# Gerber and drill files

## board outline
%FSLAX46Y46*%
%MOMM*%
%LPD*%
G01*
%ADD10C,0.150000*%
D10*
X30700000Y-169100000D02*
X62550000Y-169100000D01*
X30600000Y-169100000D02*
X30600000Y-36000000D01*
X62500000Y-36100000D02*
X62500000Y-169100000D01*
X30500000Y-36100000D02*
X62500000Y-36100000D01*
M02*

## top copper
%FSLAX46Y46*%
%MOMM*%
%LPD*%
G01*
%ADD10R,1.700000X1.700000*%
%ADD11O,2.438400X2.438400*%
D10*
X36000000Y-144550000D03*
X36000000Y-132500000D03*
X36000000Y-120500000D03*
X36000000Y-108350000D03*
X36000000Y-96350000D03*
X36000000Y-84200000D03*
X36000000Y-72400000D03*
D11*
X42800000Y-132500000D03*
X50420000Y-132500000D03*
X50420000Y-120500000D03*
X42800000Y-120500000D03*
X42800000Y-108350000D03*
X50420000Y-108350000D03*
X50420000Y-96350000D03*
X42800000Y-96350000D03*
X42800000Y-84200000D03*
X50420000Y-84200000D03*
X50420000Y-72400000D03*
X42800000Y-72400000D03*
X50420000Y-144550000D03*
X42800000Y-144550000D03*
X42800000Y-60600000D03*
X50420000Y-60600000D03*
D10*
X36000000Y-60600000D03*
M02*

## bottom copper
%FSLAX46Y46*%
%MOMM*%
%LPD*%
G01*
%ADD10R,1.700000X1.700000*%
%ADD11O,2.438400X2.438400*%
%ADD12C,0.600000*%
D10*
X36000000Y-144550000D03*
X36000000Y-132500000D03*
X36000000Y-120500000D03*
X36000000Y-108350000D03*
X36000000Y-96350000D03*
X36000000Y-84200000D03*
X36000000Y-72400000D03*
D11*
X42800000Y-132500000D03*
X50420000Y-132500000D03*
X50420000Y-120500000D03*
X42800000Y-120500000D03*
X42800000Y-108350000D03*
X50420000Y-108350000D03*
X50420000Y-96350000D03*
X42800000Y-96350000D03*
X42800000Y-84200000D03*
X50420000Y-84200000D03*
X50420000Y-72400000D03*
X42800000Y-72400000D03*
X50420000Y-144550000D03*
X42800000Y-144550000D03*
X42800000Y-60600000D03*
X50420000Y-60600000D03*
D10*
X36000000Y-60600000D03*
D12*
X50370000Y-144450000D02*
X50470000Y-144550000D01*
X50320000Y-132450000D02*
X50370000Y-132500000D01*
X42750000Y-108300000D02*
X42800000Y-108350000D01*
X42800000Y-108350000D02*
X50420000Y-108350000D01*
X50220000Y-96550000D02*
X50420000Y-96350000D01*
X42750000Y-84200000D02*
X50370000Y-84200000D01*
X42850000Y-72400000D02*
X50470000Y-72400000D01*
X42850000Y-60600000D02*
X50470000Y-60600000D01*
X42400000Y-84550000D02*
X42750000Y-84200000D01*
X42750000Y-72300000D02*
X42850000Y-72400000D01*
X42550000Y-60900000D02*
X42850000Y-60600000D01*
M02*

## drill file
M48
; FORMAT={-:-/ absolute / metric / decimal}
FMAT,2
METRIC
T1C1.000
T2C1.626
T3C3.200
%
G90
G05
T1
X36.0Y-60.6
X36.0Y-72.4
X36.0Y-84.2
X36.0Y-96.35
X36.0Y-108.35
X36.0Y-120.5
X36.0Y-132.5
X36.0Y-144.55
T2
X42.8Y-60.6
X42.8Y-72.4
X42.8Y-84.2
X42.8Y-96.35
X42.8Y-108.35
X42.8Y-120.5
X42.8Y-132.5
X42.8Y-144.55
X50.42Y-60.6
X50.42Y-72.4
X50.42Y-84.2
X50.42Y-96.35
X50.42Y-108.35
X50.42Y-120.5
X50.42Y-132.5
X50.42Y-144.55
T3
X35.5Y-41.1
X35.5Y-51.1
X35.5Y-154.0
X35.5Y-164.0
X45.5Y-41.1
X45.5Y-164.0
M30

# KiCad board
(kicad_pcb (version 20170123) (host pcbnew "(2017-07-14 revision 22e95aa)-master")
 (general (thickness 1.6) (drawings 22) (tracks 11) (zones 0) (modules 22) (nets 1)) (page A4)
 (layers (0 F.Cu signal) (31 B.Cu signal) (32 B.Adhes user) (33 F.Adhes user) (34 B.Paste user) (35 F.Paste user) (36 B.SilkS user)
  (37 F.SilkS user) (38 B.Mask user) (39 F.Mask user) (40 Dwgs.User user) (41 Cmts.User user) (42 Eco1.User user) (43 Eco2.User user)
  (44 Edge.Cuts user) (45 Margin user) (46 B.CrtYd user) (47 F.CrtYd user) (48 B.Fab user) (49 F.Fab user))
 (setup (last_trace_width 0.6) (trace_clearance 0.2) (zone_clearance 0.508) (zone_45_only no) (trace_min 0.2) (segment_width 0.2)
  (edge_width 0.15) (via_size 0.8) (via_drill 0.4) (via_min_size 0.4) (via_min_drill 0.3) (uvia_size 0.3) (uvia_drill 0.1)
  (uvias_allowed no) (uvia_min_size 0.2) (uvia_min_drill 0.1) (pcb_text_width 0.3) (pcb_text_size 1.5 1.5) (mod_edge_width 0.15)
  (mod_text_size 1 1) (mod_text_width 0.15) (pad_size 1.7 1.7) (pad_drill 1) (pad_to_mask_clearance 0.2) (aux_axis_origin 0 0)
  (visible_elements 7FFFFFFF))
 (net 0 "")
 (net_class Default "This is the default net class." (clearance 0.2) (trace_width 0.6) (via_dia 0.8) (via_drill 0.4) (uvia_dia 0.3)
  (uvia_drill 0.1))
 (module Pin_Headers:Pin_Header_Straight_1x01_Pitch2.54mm (layer F.Cu) (at 36 144.55)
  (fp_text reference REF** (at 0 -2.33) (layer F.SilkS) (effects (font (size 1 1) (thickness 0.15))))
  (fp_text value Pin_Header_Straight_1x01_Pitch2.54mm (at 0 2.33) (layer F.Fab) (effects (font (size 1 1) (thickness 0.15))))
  (pad 1 thru_hole rect (at 0 0) (size 1.7 1.7) (drill 1) (layers *.Cu *.Mask)))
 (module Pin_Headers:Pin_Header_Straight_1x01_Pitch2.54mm (layer F.Cu) (at 36 132.5)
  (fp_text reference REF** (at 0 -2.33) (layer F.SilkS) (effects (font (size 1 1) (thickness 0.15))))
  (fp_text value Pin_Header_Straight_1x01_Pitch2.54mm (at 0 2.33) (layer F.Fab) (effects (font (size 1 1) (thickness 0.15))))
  (pad 1 thru_hole rect (at 0 0) (size 1.7 1.7) (drill 1) (layers *.Cu *.Mask)))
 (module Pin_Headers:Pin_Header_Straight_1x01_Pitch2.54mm (layer F.Cu) (at 36 120.5)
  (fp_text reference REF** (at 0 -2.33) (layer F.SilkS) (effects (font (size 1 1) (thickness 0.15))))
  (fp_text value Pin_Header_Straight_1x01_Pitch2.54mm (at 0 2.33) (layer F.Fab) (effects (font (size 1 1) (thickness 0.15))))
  (pad 1 thru_hole rect (at 0 0) (size 1.7 1.7) (drill 1) (layers *.Cu *.Mask)))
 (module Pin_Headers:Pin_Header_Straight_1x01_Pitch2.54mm (layer F.Cu) (at 36 108.35)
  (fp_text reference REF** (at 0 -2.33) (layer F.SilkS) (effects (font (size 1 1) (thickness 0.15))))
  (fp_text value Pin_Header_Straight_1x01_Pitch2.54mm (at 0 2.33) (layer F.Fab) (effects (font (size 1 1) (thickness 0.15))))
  (pad 1 thru_hole rect (at 0 0) (size 1.7 1.7) (drill 1) (layers *.Cu *.Mask)))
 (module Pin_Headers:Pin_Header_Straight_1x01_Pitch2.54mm (layer F.Cu) (at 36 96.35)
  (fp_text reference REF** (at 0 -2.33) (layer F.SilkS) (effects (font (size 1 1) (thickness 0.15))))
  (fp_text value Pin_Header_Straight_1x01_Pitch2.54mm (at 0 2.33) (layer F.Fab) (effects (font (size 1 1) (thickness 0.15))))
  (pad 1 thru_hole rect (at 0 0) (size 1.7 1.7) (drill 1) (layers *.Cu *.Mask)))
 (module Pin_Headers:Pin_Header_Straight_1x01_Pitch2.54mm (layer F.Cu) (at 36 84.2)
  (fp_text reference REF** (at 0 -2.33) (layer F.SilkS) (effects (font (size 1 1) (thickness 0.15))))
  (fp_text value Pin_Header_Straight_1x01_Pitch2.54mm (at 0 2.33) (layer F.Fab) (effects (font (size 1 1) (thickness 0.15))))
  (pad 1 thru_hole rect (at 0 0) (size 1.7 1.7) (drill 1) (layers *.Cu *.Mask)))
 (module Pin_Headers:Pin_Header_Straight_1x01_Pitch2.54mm (layer F.Cu) (at 36 72.4)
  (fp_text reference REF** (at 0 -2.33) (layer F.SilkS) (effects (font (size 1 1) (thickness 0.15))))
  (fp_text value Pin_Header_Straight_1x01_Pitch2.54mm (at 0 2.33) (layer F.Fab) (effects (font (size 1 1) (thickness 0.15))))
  (pad 1 thru_hole rect (at 0 0) (size 1.7 1.7) (drill 1) (layers *.Cu *.Mask)))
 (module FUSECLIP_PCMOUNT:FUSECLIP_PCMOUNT (layer F.Cu) (at 42.8 132.5)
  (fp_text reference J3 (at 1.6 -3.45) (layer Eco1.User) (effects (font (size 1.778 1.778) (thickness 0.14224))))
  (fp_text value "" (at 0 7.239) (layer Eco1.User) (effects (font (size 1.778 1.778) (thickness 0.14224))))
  (pad 1 thru_hole oval (at 0 0) (size 2.4384 2.4384) (drill 1.6256) (layers *.Cu *.Mask))
  (pad 2 thru_hole oval (at 7.62 0) (size 2.4384 2.4384) (drill 1.6256) (layers *.Cu *.Mask)))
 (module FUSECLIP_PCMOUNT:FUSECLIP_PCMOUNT (layer F.Cu) (at 42.8 120.5)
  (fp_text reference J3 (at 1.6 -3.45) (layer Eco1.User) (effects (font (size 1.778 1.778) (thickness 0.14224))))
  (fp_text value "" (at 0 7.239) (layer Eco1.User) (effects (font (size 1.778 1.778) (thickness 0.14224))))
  (pad 2 thru_hole oval (at 7.62 0) (size 2.4384 2.4384) (drill 1.6256) (layers *.Cu *.Mask))
  (pad 1 thru_hole oval (at 0 0) (size 2.4384 2.4384) (drill 1.6256) (layers *.Cu *.Mask)))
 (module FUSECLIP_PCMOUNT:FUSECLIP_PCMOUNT (layer F.Cu) (at 42.8 108.35)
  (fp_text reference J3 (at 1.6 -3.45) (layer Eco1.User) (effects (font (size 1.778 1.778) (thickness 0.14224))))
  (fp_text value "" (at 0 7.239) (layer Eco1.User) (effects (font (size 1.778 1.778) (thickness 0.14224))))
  (pad 1 thru_hole oval (at 0 0) (size 2.4384 2.4384) (drill 1.6256) (layers *.Cu *.Mask))
  (pad 2 thru_hole oval (at 7.62 0) (size 2.4384 2.4384) (drill 1.6256) (layers *.Cu *.Mask)))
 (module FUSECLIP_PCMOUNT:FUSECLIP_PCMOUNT (layer F.Cu) (at 42.8 96.35)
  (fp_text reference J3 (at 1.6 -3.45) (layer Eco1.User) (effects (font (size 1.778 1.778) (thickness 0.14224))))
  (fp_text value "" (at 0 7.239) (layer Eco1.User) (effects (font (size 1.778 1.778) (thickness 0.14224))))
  (pad 2 thru_hole oval (at 7.62 0) (size 2.4384 2.4384) (drill 1.6256) (layers *.Cu *.Mask))
  (pad 1 thru_hole oval (at 0 0) (size 2.4384 2.4384) (drill 1.6256) (layers *.Cu *.Mask)))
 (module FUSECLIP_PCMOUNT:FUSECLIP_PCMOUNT (layer F.Cu) (at 42.8 84.2)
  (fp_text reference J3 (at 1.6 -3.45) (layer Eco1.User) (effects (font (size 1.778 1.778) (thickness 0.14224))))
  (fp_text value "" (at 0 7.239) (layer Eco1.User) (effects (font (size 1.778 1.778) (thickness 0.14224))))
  (pad 1 thru_hole oval (at 0 0) (size 2.4384 2.4384) (drill 1.6256) (layers *.Cu *.Mask))
  (pad 2 thru_hole oval (at 7.62 0) (size 2.4384 2.4384) (drill 1.6256) (layers *.Cu *.Mask)))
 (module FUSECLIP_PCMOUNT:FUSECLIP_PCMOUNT (layer F.Cu) (at 42.8 72.4)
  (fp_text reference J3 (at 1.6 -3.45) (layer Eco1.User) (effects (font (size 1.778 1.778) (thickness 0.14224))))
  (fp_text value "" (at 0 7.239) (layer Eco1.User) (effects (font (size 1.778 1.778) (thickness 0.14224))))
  (pad 2 thru_hole oval (at 7.62 0) (size 2.4384 2.4384) (drill 1.6256) (layers *.Cu *.Mask))
  (pad 1 thru_hole oval (at 0 0) (size 2.4384 2.4384) (drill 1.6256) (layers *.Cu *.Mask)))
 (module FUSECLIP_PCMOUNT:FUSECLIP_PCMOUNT (layer F.Cu) (at 42.8 144.55)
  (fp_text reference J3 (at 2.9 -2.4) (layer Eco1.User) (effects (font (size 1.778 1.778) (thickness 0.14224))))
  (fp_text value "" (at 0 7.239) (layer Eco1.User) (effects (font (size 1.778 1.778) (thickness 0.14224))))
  (pad 2 thru_hole oval (at 7.62 0) (size 2.4384 2.4384) (drill 1.6256) (layers *.Cu *.Mask))
  (pad 1 thru_hole oval (at 0 0) (size 2.4384 2.4384) (drill 1.6256) (layers *.Cu *.Mask)))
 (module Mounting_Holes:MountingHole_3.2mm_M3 (layer F.Cu) (at 35.5 154)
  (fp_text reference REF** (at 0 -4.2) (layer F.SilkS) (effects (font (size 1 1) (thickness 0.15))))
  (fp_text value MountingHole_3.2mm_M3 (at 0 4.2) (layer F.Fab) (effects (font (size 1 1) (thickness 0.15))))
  (pad "" np_thru_hole circle (at 0 0) (size 3.2 3.2) (drill 3.2) (layers *.Cu *.Mask)))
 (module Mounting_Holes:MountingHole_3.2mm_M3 (layer F.Cu) (at 35.4 51.1)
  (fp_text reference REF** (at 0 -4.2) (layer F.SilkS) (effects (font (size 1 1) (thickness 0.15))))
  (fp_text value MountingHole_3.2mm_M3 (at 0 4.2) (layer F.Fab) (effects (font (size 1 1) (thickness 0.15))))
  (pad "" np_thru_hole circle (at 0.1 0) (size 3.2 3.2) (drill 3.2) (layers *.Cu *.Mask)))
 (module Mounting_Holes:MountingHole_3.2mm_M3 (layer F.Cu) (at 45.5 164)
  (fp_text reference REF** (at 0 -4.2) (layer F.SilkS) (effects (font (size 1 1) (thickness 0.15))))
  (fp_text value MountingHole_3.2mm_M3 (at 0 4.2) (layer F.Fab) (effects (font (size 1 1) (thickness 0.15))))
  (pad "" np_thru_hole circle (at 0 0) (size 3.2 3.2) (drill 3.2) (layers *.Cu *.Mask)))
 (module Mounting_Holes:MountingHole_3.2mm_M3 (layer F.Cu) (at 35.5 41.1)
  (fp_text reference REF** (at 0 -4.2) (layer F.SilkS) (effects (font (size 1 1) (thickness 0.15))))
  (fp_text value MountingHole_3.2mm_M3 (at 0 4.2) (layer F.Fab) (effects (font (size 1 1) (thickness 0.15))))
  (pad 1 np_thru_hole circle (at 0 0) (size 3.2 3.2) (drill 3.2) (layers *.Cu *.Mask)))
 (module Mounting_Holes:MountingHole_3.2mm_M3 (layer F.Cu) (at 35.65 164)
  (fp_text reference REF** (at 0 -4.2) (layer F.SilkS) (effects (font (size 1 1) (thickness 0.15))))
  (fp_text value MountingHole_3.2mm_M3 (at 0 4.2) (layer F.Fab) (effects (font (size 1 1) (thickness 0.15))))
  (pad "" np_thru_hole circle (at -0.15 0) (size 3.2 3.2) (drill 3.2) (layers *.Cu *.Mask)))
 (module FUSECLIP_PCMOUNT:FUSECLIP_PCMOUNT (layer F.Cu) (at 42.8 60.6)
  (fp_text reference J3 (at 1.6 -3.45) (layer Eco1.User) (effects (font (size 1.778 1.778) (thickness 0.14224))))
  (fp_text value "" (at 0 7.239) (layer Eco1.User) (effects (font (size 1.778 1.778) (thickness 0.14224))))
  (pad 1 thru_hole oval (at 0 0) (size 2.4384 2.4384) (drill 1.6256) (layers *.Cu *.Mask))
  (pad 2 thru_hole oval (at 7.62 0) (size 2.4384 2.4384) (drill 1.6256) (layers *.Cu *.Mask)))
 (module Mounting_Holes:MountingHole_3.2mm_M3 (layer F.Cu) (at 45.5 41.2)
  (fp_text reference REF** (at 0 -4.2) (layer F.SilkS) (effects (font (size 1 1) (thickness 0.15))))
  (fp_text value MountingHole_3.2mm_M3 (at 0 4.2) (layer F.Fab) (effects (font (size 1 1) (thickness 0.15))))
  (pad "" np_thru_hole circle (at 0 -0.1) (size 3.2 3.2) (drill 3.2) (layers *.Cu *.Mask)))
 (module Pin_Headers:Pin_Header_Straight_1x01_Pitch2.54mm (layer F.Cu) (at 35.9 60.6)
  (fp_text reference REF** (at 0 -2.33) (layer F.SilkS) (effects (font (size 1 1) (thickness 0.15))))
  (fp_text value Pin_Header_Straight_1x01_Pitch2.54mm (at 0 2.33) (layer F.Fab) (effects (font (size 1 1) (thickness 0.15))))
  (pad 1 thru_hole rect (at 0.1 0) (size 1.7 1.7) (drill 1) (layers *.Cu *.Mask)))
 (gr_line (start 30.7 169.1) (end 62.55 169.1) (angle 90) (layer Edge.Cuts) (width 0.15))
 (gr_line (start 30.6 169.1) (end 30.6 36) (angle 90) (layer Edge.Cuts) (width 0.15))
 (gr_line (start 62.5 36.1) (end 62.5 169.1) (angle 90) (layer Edge.Cuts) (width 0.15))
 (gr_line (start 30.5 36.1) (end 62.5 36.1) (angle 90) (layer Edge.Cuts) (width 0.15))
 (segment (start 50.37 144.45) (end 50.47 144.55) (width 0.6) (layer B.Cu) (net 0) (status C00000))
 (segment (start 50.32 132.45) (end 50.37 132.5) (width 0.6) (layer B.Cu) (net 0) (status C00000))
 (segment (start 42.75 108.3) (end 42.8 108.35) (width 0.6) (layer B.Cu) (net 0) (status C00000))
 (segment (start 42.8 108.35) (end 50.42 108.35) (width 0.6) (layer B.Cu) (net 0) (status C00000))
 (segment (start 50.22 96.55) (end 50.42 96.35) (width 0.6) (layer B.Cu) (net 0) (status C00000))
 (segment (start 42.75 84.2) (end 50.37 84.2) (width 0.6) (layer B.Cu) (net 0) (status C00000))
 (segment (start 42.85 72.4) (end 50.47 72.4) (width 0.6) (layer B.Cu) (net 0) (status C00000))
 (segment (start 42.85 60.6) (end 50.47 60.6) (width 0.6) (layer B.Cu) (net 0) (status C00000))
 (segment (start 42.4 84.55) (end 42.75 84.2) (width 0.6) (layer B.Cu) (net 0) (status C00000))
 (segment (start 42.75 72.3) (end 42.85 72.4) (width 0.6) (layer B.Cu) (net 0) (status C00000))
 (segment (start 42.55 60.9) (end 42.85 60.6) (width 0.6) (layer B.Cu) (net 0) (status C00000)))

